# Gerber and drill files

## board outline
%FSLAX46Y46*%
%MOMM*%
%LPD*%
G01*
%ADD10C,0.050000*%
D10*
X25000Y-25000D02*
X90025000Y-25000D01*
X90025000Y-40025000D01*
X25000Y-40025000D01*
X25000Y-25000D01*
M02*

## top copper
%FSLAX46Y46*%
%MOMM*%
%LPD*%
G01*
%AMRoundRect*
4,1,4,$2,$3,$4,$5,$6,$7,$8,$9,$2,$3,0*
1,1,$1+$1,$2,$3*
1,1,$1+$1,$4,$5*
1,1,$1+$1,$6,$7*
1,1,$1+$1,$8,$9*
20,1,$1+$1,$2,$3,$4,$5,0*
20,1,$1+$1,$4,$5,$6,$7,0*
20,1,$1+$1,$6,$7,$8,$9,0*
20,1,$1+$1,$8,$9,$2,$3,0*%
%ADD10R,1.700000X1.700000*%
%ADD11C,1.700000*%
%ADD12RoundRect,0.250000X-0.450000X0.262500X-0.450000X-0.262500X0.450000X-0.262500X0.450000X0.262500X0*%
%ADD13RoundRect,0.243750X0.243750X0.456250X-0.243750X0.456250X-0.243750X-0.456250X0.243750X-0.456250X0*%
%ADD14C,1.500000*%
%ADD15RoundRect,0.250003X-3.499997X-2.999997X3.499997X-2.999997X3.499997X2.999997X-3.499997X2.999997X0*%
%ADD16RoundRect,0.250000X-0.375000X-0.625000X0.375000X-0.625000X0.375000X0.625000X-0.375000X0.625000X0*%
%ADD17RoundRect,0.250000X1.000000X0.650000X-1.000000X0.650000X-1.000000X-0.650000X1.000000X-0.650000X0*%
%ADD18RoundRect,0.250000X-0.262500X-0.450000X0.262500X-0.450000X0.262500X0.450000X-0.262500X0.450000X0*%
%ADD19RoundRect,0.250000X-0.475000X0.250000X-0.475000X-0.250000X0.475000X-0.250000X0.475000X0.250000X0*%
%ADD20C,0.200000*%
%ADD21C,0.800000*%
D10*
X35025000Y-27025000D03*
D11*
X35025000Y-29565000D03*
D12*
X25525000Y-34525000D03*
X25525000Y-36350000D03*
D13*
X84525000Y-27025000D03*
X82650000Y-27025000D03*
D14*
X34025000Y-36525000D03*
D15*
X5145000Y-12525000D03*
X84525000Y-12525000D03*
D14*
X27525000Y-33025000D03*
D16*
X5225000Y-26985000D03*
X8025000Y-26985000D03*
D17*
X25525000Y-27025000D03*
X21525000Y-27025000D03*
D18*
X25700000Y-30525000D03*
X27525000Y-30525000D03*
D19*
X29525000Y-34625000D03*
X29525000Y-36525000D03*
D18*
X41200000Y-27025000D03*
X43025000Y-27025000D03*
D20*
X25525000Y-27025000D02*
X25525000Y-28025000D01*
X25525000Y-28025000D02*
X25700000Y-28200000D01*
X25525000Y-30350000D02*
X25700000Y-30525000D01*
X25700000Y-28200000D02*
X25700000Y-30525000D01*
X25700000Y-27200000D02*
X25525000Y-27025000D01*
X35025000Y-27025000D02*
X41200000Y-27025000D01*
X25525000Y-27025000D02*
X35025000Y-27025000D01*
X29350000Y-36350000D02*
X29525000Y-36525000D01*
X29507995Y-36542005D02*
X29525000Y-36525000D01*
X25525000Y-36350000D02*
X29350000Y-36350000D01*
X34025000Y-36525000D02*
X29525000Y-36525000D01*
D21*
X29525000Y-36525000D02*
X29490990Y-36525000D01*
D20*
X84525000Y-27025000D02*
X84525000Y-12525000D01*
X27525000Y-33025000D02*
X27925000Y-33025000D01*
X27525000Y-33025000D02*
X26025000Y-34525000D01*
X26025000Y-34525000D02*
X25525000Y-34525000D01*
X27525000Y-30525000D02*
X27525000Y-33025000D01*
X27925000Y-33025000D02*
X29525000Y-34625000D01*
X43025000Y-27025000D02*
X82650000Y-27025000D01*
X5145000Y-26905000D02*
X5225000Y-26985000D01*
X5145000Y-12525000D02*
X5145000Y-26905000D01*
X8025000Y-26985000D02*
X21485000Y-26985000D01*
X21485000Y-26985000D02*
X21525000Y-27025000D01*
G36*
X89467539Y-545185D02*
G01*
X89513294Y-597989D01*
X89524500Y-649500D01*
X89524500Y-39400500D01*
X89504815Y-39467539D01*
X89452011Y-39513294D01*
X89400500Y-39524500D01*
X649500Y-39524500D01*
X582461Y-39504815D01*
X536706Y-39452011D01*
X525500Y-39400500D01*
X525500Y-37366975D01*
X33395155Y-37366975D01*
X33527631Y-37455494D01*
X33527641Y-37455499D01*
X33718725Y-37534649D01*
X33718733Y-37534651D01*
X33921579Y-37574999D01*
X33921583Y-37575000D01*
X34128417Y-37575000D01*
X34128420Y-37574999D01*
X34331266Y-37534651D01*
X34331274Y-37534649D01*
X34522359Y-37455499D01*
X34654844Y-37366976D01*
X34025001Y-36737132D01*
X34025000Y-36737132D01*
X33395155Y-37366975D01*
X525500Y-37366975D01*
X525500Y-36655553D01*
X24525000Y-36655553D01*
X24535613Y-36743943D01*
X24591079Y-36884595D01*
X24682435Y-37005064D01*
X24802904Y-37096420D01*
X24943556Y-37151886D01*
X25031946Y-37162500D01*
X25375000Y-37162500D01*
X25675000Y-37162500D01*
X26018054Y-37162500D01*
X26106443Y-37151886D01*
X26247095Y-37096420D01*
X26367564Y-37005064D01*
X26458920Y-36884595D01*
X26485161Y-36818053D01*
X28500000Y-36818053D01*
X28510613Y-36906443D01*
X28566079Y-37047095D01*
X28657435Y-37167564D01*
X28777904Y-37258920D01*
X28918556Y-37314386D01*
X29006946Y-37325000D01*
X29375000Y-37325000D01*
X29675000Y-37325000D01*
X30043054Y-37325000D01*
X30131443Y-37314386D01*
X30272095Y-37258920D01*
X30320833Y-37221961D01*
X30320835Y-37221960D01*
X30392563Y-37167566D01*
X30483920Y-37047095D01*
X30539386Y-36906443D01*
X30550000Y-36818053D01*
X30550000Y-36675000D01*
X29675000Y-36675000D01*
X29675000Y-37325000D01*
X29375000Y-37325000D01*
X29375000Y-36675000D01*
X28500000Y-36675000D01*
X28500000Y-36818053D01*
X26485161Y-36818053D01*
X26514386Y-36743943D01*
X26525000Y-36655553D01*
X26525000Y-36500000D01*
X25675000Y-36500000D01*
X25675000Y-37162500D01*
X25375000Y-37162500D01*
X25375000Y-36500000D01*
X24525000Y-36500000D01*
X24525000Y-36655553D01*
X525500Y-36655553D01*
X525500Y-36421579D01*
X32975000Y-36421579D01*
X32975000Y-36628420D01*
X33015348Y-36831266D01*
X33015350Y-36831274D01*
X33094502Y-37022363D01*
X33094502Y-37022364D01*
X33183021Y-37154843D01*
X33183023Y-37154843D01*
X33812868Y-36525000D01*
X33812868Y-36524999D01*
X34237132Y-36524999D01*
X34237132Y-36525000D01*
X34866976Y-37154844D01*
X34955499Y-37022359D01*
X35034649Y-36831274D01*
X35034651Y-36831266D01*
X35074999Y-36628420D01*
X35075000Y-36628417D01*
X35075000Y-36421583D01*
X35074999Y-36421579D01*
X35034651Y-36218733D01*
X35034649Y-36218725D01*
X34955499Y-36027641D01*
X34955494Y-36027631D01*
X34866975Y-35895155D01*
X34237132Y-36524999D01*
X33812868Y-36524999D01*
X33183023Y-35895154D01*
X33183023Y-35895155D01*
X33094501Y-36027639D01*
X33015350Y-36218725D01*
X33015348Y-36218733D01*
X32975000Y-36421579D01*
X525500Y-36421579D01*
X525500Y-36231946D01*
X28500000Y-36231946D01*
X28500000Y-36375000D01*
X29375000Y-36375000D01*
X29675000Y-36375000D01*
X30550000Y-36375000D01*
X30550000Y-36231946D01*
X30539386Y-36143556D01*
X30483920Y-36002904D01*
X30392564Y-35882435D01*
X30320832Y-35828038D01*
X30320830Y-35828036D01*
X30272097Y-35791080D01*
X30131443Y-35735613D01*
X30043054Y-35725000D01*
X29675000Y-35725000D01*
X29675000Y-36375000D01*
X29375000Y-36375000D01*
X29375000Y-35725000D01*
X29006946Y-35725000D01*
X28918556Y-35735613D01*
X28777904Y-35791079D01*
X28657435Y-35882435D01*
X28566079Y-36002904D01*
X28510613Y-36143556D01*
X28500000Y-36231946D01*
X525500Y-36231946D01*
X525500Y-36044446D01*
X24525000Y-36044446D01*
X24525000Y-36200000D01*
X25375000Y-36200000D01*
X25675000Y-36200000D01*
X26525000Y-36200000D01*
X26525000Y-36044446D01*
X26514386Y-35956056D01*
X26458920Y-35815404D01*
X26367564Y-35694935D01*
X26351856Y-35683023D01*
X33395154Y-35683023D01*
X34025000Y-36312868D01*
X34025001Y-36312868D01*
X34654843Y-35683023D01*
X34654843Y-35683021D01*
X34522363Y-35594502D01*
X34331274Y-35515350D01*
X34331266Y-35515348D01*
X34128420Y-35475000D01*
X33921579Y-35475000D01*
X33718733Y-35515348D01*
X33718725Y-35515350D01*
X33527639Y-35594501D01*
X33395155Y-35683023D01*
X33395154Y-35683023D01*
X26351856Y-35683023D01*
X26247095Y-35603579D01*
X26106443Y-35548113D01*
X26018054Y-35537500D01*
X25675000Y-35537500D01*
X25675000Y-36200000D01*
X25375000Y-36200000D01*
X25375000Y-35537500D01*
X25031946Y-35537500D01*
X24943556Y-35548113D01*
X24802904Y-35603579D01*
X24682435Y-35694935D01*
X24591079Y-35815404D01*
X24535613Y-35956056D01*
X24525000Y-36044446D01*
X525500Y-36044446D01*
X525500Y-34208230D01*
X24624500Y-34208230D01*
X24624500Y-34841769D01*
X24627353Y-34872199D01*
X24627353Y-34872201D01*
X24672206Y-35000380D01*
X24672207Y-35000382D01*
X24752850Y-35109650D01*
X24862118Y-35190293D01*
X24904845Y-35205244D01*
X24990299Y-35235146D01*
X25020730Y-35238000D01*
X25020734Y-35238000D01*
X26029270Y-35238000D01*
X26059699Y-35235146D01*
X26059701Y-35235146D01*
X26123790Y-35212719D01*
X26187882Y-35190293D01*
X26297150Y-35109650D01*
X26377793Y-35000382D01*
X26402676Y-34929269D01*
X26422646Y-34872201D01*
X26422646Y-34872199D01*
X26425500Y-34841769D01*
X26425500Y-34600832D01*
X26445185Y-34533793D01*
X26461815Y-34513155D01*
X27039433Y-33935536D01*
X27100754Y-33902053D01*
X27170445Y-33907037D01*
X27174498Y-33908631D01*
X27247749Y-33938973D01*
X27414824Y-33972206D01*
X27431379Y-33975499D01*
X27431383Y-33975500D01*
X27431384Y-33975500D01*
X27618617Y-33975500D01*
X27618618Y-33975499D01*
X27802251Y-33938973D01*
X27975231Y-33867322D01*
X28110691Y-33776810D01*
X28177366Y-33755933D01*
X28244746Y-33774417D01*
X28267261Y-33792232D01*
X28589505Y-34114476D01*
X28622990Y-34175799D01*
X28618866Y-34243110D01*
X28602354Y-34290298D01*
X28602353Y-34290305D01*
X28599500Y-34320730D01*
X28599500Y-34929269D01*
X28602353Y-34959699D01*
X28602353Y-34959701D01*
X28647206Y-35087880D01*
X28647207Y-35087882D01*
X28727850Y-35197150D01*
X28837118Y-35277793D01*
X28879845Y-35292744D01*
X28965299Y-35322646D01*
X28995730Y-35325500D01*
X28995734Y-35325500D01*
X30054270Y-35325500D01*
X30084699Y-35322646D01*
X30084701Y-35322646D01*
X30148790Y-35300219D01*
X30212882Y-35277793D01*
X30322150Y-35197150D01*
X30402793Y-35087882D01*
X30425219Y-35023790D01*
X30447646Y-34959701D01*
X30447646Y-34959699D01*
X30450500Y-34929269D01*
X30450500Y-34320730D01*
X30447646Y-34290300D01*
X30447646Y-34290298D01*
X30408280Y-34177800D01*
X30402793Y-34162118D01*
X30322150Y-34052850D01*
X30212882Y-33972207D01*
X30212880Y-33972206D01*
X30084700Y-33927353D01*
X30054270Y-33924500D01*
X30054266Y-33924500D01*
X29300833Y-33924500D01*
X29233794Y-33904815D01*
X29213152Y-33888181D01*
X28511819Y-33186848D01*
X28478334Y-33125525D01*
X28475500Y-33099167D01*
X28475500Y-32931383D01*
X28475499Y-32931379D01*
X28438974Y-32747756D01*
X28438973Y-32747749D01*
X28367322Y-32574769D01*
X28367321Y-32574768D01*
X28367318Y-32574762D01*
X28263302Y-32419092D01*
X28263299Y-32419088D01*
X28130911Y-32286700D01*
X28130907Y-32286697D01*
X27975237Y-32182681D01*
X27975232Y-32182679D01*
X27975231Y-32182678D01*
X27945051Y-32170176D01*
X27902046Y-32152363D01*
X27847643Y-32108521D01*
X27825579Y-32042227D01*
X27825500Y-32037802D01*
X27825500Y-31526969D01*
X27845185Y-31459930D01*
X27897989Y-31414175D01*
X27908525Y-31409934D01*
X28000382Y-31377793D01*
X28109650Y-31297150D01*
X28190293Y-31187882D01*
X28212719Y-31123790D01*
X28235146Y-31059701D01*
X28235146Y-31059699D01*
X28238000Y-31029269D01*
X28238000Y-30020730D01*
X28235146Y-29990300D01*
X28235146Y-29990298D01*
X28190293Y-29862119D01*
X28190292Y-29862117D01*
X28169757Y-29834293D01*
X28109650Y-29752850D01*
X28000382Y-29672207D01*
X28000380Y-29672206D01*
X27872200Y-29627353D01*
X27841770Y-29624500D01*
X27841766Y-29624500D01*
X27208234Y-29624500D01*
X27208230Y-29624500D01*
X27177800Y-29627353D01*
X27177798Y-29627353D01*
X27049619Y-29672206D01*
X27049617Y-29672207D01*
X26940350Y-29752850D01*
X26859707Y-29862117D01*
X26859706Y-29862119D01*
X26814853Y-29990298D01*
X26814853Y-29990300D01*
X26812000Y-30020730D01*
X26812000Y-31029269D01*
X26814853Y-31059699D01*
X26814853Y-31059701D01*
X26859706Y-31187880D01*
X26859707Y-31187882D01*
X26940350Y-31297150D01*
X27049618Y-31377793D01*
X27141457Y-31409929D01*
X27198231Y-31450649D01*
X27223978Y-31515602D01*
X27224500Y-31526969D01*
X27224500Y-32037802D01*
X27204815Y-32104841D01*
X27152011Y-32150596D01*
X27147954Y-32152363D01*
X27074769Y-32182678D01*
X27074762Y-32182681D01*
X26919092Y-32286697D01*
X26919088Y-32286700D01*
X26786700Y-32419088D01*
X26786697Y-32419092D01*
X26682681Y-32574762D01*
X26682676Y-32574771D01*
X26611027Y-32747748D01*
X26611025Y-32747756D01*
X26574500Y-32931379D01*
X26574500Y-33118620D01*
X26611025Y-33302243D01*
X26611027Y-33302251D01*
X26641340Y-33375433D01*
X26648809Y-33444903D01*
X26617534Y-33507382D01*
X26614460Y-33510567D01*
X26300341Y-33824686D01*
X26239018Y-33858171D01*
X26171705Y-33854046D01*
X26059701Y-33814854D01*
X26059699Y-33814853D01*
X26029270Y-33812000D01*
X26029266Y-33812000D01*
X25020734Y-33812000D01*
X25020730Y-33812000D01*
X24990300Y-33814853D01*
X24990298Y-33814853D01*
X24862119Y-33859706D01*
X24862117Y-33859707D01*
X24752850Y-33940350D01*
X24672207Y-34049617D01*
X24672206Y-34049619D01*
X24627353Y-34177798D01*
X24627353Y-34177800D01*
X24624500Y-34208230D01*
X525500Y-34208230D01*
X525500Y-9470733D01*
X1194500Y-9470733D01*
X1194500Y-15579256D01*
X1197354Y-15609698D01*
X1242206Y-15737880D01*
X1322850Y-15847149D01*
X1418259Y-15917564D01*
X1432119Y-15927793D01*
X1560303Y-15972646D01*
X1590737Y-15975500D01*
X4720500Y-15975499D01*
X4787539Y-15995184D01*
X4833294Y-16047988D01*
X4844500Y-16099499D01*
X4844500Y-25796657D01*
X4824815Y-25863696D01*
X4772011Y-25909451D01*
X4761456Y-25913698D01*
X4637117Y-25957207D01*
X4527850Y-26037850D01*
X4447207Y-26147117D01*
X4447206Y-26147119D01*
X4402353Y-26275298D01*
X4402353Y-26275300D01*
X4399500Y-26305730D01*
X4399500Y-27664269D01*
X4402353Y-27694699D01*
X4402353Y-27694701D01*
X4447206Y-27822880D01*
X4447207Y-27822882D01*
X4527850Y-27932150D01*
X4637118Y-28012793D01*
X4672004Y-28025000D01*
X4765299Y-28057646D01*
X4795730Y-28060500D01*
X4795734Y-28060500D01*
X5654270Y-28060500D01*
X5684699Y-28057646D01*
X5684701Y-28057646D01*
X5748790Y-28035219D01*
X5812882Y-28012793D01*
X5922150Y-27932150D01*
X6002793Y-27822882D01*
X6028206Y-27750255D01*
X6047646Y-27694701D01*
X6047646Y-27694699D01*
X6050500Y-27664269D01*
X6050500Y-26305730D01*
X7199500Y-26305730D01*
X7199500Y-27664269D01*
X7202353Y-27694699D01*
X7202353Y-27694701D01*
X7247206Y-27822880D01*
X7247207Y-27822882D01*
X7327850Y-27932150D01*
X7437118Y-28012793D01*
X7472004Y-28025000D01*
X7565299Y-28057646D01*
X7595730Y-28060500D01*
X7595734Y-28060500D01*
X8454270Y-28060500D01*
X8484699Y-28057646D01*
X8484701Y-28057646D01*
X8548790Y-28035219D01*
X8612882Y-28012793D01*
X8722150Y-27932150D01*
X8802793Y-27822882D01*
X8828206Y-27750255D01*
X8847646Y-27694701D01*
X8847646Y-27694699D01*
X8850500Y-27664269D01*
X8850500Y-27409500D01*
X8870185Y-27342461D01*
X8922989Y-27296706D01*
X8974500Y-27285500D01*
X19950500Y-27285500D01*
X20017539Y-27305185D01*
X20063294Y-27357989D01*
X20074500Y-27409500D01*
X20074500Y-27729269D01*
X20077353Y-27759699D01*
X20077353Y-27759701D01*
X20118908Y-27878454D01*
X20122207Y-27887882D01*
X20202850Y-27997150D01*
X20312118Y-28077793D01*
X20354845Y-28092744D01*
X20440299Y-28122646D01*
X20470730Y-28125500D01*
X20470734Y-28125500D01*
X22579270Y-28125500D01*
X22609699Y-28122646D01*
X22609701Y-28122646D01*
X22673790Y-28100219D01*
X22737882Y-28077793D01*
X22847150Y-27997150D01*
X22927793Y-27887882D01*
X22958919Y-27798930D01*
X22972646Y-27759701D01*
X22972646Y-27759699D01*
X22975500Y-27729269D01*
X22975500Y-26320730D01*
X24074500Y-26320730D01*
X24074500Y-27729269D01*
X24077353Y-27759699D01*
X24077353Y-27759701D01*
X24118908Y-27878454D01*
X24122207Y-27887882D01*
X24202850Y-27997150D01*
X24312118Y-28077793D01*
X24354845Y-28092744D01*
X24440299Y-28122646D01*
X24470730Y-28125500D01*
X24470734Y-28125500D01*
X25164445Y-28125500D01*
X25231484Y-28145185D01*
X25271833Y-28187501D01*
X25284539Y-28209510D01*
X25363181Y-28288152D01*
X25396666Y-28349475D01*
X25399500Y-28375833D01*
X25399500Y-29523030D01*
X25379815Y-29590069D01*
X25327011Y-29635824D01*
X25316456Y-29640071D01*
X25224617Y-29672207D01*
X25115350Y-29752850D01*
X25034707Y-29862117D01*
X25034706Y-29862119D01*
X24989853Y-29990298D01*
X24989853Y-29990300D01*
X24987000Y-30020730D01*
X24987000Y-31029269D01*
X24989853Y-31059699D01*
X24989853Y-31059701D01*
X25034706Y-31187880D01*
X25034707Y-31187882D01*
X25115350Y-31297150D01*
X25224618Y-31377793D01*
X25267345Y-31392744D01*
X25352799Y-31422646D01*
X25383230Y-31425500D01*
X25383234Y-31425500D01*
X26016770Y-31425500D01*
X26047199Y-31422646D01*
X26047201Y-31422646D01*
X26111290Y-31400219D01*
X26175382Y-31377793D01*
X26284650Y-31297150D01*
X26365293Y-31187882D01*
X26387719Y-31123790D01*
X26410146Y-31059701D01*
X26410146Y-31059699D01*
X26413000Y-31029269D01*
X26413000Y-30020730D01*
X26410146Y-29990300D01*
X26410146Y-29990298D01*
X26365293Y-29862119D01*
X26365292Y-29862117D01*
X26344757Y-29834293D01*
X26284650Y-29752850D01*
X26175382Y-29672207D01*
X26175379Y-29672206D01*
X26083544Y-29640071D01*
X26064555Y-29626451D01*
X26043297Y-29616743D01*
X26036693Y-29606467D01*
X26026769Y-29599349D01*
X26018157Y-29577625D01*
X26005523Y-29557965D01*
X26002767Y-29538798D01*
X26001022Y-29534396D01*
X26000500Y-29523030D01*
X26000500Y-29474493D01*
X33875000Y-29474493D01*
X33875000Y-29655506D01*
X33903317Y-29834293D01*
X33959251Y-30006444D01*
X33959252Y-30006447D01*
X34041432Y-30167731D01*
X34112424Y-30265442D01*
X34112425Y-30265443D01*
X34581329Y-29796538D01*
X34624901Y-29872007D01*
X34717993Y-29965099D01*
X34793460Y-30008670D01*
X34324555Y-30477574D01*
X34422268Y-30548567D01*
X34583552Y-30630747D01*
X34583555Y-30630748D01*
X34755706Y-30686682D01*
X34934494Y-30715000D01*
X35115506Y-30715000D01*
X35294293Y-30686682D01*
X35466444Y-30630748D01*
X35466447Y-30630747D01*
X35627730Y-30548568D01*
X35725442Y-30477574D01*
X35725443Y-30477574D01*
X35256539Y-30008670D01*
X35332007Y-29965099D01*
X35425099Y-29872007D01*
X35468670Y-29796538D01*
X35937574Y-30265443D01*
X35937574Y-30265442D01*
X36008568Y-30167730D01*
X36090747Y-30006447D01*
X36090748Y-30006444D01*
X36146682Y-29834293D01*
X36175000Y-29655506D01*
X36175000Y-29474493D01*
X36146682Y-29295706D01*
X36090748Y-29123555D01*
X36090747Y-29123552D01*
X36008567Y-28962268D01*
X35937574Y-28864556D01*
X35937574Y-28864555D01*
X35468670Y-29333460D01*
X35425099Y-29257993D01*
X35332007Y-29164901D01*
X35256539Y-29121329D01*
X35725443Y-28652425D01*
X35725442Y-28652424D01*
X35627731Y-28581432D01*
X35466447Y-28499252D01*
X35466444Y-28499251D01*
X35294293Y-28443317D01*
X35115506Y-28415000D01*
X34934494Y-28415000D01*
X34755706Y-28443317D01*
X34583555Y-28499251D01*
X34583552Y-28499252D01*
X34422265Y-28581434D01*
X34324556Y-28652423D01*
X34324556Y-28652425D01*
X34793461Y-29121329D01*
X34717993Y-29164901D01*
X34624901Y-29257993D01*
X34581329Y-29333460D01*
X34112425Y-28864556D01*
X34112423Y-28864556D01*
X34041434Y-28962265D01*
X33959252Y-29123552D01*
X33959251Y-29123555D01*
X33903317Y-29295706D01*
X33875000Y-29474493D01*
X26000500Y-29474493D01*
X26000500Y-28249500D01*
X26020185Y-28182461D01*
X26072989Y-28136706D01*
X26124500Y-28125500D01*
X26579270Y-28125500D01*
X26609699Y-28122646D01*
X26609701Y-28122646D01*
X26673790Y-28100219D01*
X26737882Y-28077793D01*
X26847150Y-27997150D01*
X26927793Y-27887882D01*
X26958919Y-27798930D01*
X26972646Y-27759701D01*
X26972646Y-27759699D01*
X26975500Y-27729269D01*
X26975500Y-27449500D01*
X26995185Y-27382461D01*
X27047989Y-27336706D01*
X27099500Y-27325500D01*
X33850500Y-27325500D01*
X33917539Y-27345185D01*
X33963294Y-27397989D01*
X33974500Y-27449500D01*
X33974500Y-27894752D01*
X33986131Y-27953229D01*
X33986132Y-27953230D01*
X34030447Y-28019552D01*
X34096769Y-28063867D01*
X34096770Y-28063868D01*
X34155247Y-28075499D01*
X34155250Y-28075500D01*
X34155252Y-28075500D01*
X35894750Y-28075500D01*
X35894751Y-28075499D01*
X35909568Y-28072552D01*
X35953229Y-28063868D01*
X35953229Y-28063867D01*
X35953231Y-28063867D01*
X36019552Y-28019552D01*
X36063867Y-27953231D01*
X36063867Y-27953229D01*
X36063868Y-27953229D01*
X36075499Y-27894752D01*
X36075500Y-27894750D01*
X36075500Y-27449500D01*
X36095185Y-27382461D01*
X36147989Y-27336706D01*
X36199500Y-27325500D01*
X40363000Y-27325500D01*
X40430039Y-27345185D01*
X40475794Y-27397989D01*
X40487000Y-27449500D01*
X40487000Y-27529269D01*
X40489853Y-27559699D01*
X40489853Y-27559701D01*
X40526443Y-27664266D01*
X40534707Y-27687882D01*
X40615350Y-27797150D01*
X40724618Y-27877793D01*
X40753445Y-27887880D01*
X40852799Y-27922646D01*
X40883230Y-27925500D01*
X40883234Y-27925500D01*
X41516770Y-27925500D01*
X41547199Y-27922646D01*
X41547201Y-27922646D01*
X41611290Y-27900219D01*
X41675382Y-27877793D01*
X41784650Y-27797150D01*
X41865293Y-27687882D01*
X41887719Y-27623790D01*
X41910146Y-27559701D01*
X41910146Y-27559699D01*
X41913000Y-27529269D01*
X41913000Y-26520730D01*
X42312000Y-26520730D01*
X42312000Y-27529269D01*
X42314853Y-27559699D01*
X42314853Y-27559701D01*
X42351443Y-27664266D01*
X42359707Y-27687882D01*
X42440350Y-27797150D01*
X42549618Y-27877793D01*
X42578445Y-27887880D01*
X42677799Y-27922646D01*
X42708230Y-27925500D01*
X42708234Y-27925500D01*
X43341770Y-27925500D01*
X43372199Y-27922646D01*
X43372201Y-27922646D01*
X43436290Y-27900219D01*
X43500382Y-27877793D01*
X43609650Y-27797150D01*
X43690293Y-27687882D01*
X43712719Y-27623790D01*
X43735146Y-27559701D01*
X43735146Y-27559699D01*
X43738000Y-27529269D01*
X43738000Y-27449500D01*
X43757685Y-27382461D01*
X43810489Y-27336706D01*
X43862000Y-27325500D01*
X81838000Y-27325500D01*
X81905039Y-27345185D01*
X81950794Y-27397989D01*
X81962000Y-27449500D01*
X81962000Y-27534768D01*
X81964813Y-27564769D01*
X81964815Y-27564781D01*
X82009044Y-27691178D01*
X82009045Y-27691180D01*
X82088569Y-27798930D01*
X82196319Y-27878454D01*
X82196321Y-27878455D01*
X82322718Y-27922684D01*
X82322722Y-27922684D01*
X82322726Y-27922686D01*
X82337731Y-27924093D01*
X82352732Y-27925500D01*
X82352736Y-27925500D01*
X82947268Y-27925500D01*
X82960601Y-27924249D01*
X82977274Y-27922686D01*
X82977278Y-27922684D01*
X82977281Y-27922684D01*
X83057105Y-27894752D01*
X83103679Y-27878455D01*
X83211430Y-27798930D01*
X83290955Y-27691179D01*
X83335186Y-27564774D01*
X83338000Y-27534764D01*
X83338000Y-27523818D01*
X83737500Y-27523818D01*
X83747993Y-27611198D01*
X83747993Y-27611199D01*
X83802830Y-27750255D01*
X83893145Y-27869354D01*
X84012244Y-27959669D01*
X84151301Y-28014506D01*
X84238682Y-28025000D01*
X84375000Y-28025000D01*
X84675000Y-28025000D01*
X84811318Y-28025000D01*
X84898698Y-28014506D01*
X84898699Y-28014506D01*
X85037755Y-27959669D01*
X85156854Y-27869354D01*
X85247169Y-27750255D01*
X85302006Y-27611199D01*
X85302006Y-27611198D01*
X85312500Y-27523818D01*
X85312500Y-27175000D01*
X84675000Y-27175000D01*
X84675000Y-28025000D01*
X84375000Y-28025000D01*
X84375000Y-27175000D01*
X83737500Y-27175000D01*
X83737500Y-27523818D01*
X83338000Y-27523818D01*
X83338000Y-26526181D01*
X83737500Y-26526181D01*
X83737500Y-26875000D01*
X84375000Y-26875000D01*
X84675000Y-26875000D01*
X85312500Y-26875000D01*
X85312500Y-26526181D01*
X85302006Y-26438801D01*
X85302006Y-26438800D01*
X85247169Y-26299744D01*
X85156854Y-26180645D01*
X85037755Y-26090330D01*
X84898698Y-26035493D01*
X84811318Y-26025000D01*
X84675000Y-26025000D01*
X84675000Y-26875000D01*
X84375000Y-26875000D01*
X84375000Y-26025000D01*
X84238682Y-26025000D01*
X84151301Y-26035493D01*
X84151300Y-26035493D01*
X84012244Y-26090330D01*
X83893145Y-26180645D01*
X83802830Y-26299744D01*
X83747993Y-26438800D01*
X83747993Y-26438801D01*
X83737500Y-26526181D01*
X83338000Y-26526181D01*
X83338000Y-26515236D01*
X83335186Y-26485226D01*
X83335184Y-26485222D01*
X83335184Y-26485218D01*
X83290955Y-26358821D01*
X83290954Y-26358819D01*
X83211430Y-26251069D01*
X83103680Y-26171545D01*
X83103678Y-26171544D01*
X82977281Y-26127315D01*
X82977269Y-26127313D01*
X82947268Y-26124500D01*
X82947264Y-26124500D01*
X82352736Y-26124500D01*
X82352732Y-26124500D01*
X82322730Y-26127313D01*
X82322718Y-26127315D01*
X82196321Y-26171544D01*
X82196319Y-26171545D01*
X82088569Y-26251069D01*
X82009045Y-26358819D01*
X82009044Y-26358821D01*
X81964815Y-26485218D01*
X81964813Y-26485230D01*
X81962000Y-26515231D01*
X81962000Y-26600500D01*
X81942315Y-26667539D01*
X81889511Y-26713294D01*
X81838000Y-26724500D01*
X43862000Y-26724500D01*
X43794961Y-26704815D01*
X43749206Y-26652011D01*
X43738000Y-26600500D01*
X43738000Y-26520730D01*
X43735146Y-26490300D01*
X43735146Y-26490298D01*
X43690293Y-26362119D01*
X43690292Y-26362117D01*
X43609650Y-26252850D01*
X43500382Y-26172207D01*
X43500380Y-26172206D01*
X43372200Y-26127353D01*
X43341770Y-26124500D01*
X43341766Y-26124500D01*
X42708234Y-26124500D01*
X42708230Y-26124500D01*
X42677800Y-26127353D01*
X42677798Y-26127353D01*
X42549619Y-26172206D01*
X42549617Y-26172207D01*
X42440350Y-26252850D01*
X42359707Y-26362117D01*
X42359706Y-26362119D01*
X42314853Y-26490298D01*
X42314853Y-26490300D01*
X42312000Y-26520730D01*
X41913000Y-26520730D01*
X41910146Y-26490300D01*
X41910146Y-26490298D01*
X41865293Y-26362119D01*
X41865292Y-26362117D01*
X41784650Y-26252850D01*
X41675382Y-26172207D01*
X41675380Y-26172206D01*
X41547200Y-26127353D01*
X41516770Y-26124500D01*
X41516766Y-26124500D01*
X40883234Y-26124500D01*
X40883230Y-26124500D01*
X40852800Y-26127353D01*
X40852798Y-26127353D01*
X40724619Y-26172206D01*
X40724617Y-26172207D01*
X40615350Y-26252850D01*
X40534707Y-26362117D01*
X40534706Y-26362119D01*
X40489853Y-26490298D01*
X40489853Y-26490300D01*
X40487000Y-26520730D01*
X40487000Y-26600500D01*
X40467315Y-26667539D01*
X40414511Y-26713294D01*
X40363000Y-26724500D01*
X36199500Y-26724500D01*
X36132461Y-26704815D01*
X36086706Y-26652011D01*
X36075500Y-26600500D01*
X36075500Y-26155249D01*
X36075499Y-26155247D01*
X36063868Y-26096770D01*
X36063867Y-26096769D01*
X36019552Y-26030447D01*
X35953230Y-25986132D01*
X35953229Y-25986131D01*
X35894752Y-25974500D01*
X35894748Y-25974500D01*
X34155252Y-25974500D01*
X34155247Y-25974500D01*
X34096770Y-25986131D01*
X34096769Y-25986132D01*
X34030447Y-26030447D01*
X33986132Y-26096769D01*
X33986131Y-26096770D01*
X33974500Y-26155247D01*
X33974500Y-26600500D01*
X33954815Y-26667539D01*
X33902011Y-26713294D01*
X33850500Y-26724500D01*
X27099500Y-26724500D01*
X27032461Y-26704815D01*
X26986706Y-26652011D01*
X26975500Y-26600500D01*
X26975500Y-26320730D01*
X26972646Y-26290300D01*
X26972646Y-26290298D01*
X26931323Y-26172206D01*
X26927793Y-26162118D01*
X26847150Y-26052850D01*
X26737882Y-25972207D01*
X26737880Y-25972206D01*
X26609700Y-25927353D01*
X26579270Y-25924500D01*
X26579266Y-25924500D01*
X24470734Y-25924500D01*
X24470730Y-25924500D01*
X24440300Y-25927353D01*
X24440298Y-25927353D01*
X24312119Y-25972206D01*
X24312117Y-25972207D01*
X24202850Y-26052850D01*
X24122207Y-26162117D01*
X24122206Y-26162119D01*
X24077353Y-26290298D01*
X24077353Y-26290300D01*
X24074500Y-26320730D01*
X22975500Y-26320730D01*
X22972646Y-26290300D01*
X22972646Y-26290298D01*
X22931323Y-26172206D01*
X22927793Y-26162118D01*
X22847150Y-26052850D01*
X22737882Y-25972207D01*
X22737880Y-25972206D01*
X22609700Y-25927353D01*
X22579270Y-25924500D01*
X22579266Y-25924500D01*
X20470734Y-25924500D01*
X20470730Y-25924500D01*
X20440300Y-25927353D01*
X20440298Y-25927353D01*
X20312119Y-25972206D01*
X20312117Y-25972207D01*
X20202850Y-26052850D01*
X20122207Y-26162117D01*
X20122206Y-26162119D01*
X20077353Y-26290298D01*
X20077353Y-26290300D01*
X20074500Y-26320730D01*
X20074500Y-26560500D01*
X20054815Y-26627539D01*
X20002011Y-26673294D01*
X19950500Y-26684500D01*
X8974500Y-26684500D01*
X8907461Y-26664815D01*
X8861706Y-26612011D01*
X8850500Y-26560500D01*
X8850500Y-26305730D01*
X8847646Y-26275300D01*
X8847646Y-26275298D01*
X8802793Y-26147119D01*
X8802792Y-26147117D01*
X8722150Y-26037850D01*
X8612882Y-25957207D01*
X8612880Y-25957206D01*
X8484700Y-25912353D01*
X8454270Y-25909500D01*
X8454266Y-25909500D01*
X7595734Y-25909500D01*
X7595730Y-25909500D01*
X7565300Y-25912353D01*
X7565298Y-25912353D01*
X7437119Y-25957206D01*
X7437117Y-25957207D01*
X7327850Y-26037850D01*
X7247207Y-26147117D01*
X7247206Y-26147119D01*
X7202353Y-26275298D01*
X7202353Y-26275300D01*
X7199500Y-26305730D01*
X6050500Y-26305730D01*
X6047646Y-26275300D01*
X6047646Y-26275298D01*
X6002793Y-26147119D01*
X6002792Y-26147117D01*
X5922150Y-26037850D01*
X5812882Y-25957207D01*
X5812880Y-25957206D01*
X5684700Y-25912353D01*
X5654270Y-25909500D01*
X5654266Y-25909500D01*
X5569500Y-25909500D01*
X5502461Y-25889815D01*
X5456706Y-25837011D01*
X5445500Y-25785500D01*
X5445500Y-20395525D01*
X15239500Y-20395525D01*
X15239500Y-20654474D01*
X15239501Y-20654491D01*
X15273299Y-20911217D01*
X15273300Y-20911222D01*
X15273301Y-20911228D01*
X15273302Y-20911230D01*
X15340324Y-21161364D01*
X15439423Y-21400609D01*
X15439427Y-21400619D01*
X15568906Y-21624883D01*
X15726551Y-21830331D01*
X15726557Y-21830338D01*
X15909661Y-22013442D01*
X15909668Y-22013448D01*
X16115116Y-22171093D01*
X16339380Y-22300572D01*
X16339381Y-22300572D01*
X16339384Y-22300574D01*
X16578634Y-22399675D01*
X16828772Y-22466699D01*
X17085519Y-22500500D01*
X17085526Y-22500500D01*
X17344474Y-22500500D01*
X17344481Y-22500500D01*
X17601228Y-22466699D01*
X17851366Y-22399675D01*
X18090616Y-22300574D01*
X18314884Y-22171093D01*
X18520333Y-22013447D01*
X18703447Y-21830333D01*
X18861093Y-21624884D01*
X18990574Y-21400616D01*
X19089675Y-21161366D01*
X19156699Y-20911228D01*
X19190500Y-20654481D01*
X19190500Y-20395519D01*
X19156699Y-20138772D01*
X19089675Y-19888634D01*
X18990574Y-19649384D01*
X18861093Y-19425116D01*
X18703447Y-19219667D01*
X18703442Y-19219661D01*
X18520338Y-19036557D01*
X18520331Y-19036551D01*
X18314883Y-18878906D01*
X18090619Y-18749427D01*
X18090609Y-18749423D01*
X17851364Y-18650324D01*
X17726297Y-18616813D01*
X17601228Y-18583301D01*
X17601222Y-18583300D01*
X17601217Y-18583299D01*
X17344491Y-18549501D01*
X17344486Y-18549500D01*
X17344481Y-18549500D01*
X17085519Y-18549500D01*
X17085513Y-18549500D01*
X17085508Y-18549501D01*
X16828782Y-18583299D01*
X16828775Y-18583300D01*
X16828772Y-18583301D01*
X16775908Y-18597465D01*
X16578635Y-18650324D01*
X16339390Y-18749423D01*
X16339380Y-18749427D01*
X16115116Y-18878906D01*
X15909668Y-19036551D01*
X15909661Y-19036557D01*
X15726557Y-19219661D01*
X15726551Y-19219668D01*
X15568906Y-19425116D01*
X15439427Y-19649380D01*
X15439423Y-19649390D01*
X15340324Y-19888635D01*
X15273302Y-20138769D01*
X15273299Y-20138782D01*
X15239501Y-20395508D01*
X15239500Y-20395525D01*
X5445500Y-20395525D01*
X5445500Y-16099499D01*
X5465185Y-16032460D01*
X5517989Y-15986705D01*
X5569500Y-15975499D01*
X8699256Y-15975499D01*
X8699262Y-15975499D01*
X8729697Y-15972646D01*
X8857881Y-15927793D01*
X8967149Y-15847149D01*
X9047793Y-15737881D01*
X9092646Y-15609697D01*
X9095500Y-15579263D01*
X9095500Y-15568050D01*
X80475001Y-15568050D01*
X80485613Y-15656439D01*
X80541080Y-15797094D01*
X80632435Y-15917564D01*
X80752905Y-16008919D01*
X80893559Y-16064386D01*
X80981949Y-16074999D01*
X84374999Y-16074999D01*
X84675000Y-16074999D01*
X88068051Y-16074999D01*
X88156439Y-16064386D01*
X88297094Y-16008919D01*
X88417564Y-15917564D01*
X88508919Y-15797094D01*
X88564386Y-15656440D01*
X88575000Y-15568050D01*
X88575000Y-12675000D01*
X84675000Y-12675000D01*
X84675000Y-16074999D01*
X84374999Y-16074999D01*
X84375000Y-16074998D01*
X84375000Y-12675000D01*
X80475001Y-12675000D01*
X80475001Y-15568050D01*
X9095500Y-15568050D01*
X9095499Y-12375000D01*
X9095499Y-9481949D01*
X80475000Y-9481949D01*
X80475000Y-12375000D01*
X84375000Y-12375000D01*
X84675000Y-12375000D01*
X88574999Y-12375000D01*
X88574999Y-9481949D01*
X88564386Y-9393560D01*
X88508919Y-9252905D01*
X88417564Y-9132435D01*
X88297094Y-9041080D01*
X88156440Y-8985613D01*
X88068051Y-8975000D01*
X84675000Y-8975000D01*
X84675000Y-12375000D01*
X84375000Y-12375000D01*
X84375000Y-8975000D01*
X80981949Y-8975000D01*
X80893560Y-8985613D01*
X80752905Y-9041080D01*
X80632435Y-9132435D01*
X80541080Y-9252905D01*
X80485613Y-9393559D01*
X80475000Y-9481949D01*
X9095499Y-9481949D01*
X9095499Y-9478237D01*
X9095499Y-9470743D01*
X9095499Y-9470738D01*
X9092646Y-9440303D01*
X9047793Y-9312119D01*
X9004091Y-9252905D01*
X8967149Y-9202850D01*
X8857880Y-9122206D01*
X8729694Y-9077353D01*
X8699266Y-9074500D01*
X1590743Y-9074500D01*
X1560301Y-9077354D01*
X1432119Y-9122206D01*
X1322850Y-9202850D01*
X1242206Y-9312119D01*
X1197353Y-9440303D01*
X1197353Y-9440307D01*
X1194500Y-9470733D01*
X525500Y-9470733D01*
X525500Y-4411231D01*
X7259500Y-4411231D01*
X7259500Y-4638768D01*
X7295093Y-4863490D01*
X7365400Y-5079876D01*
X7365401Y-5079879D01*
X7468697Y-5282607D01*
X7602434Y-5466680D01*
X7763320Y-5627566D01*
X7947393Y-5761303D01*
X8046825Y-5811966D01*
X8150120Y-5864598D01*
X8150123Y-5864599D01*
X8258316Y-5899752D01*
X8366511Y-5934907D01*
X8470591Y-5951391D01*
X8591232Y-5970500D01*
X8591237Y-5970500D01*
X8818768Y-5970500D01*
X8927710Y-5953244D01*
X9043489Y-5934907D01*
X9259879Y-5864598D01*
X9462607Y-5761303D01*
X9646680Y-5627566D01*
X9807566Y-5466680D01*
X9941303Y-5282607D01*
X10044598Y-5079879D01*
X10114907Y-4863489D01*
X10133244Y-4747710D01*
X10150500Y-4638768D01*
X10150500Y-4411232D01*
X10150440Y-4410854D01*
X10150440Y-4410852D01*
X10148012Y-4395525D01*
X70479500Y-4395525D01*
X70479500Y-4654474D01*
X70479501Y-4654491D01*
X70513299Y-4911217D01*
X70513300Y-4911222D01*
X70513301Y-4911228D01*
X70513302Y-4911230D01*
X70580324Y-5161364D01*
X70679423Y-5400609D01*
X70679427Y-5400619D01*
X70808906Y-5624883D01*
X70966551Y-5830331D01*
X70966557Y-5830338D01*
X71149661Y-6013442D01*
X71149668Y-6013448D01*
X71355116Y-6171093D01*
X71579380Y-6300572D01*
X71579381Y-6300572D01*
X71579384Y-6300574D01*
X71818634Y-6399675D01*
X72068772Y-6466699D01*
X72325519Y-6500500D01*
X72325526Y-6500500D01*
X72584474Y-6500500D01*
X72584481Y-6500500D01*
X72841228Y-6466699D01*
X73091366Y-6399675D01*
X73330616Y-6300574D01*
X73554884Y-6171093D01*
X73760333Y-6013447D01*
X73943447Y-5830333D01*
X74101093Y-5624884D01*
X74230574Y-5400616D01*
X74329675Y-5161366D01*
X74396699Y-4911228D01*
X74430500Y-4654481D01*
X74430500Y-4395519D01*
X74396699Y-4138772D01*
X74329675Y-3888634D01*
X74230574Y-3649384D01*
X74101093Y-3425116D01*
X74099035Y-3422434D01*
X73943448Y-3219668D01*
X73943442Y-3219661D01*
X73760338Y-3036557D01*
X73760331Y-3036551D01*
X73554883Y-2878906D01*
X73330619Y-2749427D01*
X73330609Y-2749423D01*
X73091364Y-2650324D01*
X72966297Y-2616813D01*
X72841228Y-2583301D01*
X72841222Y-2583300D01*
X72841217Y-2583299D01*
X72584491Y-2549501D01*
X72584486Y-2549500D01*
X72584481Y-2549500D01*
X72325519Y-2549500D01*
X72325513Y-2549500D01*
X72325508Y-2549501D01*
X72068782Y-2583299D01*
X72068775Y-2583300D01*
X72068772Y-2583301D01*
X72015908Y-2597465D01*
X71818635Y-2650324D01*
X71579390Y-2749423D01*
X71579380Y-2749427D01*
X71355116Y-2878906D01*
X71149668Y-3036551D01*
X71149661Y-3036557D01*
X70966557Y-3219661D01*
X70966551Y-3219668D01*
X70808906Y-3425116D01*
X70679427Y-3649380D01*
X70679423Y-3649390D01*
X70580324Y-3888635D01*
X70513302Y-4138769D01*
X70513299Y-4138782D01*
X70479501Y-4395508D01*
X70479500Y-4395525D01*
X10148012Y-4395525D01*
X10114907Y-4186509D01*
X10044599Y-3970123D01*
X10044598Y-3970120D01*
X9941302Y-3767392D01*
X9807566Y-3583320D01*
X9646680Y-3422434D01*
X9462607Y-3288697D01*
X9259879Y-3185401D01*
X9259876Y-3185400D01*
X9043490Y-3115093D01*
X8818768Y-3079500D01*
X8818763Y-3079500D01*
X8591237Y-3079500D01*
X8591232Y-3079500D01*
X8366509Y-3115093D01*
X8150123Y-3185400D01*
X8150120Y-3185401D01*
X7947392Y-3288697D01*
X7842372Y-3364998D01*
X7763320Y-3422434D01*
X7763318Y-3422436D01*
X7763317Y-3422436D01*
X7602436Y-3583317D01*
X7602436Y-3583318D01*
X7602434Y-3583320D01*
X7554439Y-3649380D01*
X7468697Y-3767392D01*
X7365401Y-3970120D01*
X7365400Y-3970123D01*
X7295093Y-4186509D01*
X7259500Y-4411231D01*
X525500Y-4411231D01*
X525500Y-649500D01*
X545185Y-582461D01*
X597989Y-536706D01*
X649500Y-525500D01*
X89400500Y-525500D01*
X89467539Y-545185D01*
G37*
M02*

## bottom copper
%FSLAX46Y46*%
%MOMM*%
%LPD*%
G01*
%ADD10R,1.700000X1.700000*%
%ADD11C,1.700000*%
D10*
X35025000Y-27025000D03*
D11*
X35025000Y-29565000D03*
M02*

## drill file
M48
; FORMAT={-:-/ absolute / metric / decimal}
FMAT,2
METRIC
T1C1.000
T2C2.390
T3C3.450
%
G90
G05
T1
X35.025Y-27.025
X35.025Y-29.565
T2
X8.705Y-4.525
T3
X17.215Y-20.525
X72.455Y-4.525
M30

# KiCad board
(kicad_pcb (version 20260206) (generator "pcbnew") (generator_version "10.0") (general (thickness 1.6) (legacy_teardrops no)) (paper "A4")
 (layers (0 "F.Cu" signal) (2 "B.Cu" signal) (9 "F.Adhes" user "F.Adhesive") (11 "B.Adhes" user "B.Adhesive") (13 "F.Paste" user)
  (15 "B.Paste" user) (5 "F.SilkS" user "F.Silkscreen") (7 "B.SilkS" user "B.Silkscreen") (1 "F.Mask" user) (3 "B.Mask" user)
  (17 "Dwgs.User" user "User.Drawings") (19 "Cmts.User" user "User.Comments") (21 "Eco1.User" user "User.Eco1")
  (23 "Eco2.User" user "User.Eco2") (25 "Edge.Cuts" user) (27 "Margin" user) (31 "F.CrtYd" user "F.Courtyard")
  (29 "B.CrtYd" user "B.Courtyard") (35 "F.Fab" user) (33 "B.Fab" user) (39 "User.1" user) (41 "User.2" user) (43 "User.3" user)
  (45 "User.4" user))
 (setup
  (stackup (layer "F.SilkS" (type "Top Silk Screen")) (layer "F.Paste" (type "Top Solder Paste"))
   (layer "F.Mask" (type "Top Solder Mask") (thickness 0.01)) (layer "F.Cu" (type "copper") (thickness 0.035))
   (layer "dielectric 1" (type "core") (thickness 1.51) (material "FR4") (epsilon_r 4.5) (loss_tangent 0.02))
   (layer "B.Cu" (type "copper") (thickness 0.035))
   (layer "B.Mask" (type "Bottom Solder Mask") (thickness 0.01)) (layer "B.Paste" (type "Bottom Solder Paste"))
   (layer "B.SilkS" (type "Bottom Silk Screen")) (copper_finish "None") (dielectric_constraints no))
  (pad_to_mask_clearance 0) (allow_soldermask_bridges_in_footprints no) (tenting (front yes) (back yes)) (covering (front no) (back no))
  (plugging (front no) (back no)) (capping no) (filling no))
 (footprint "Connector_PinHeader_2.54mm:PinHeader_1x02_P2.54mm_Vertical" (layer "F.Cu") (at 35.025 27.025)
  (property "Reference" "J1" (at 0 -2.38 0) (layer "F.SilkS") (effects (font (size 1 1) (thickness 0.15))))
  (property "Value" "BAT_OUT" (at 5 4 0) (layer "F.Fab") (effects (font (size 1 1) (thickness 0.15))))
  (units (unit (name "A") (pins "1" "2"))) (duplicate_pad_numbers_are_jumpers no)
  (pad "1" thru_hole rect (at 0 0) (size 1.7 1.7) (drill 1) (layers "*.Cu" "*.Mask") (remove_unused_layers no) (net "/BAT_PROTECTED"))
  (pad "2" thru_hole circle (at 0 2.54) (size 1.7 1.7) (drill 1) (layers "*.Cu" "*.Mask") (remove_unused_layers no) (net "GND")))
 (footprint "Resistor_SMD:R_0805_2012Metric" (layer "F.Cu") (at 25.525 35.4375 -90)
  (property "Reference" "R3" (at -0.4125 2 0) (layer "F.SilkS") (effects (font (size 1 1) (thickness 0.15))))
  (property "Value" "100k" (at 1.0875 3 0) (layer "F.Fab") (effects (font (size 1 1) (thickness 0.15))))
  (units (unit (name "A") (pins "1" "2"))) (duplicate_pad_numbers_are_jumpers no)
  (pad "1" smd roundrect (at -0.9125 0 270) (size 1.025 1.4) (layers "F.Cu" "F.Mask" "F.Paste") (roundrect_rratio 0.243902)
   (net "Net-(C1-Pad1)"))
  (pad "2" smd roundrect (at 0.9125 0 270) (size 1.025 1.4) (layers "F.Cu" "F.Mask" "F.Paste") (roundrect_rratio 0.243902) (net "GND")))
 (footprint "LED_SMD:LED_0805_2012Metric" (layer "F.Cu") (at 83.5875 27.025 180)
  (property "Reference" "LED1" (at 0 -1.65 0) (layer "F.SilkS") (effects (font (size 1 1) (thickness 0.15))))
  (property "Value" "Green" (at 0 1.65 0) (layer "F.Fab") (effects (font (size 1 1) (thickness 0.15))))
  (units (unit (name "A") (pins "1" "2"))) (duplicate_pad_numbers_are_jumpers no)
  (pad "1" smd roundrect (at -0.9375 0 180) (size 0.975 1.4) (layers "F.Cu" "F.Mask" "F.Paste") (roundrect_rratio 0.25) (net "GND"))
  (pad "2" smd roundrect (at 0.9375 0 180) (size 0.975 1.4) (layers "F.Cu" "F.Mask" "F.Paste") (roundrect_rratio 0.25) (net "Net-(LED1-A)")))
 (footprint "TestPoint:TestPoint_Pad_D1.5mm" (layer "F.Cu") (at 34.025 36.525)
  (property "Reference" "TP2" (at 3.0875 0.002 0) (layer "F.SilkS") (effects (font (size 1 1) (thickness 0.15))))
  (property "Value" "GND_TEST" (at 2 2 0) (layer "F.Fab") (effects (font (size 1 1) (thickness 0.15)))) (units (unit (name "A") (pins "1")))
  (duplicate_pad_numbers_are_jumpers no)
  (pad "1" smd circle (at 0 0) (size 1.5 1.5) (layers "F.Cu" "F.Mask") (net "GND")))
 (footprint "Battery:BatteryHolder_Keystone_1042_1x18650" (layer "F.Cu") (at 44.835 12.525)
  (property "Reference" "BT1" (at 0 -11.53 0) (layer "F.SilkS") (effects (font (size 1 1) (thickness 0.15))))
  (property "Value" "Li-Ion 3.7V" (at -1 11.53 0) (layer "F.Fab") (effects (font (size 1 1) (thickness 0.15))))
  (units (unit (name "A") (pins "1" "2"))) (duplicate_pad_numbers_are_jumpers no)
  (pad "" np_thru_hole circle (at -36.13 -8) (size 2.39 2.39) (drill 2.39) (layers "*.Cu" "*.Mask"))
  (pad "" np_thru_hole circle (at -27.62 8) (size 3.45 3.45) (drill 3.45) (layers "*.Cu" "*.Mask"))
  (pad "" np_thru_hole circle (at 27.62 -8) (size 3.45 3.45) (drill 3.45) (layers "*.Cu" "*.Mask"))
  (pad "1" smd roundrect (at -39.69 0) (size 7.5 6.5) (layers "F.Cu" "F.Mask" "F.Paste") (roundrect_rratio 0.038462) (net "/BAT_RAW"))
  (pad "2" smd roundrect (at 39.69 0) (size 7.5 6.5) (layers "F.Cu" "F.Mask" "F.Paste") (roundrect_rratio 0.038462) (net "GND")))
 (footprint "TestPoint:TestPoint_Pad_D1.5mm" (layer "F.Cu") (at 27.525 33.025)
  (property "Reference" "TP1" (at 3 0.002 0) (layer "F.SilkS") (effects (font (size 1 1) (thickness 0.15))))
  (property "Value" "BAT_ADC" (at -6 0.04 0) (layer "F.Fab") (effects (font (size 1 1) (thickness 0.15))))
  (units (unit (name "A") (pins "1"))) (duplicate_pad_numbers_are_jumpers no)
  (pad "1" smd circle (at 0 0) (size 1.5 1.5) (layers "F.Cu" "F.Mask") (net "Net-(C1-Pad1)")))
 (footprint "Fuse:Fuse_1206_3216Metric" (layer "F.Cu") (at 6.625 26.985)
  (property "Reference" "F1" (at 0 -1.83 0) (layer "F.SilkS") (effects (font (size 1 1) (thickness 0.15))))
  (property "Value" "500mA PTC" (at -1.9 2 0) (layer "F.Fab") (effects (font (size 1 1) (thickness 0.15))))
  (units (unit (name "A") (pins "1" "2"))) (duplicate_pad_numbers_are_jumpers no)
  (pad "1" smd roundrect (at -1.4 0) (size 1.25 1.75) (layers "F.Cu" "F.Mask" "F.Paste") (roundrect_rratio 0.2) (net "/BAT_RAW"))
  (pad "2" smd roundrect (at 1.4 0) (size 1.25 1.75) (layers "F.Cu" "F.Mask" "F.Paste") (roundrect_rratio 0.2) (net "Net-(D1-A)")))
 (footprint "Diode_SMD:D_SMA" (layer "F.Cu") (at 23.525 27.025 180)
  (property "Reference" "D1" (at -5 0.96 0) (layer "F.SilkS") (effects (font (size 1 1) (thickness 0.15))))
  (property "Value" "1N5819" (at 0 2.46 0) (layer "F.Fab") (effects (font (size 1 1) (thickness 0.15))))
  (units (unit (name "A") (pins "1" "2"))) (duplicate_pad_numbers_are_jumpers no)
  (pad "1" smd roundrect (at -2 0 180) (size 2.5 1.8) (layers "F.Cu" "F.Mask" "F.Paste") (roundrect_rratio 0.1388888889)
   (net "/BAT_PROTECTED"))
  (pad "2" smd roundrect (at 2 0 180) (size 2.5 1.8) (layers "F.Cu" "F.Mask" "F.Paste") (roundrect_rratio 0.1388888889) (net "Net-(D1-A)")))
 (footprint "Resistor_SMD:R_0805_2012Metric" (layer "F.Cu") (at 26.6125 30.525)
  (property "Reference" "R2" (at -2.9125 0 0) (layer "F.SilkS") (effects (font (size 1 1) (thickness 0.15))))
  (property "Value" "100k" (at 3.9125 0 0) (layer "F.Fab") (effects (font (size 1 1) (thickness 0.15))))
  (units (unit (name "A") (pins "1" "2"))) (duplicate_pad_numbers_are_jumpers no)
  (pad "1" smd roundrect (at -0.9125 0) (size 1.025 1.4) (layers "F.Cu" "F.Mask" "F.Paste") (roundrect_rratio 0.243902)
   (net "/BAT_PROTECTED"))
  (pad "2" smd roundrect (at 0.9125 0) (size 1.025 1.4) (layers "F.Cu" "F.Mask" "F.Paste") (roundrect_rratio 0.243902) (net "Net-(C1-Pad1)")))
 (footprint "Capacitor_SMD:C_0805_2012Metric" (layer "F.Cu") (at 29.525 35.575 -90)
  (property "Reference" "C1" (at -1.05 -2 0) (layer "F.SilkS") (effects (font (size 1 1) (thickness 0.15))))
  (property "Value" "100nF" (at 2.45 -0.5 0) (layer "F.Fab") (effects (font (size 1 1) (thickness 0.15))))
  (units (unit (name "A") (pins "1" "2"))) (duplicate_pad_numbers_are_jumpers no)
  (pad "1" smd roundrect (at -0.95 0 270) (size 1 1.45) (layers "F.Cu" "F.Mask" "F.Paste") (roundrect_rratio 0.25) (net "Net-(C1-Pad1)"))
  (pad "2" smd roundrect (at 0.95 0 270) (size 1 1.45) (layers "F.Cu" "F.Mask" "F.Paste") (roundrect_rratio 0.25) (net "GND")))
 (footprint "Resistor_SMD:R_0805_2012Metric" (layer "F.Cu") (at 42.1125 27.025)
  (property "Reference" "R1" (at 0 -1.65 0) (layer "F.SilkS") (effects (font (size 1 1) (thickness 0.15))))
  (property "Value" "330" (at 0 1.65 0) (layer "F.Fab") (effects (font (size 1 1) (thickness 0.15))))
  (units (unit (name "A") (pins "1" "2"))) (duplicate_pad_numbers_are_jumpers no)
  (pad "1" smd roundrect (at -0.9125 0) (size 1.025 1.4) (layers "F.Cu" "F.Mask" "F.Paste") (roundrect_rratio 0.243902)
   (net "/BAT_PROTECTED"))
  (pad "2" smd roundrect (at 0.9125 0) (size 1.025 1.4) (layers "F.Cu" "F.Mask" "F.Paste") (roundrect_rratio 0.243902) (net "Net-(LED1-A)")))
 (gr_rect (start 0.025 0.025) (end 90.025 40.025) (stroke (width 0.05) (type default)) (fill no) (layer "Edge.Cuts"))
 (segment (start 25.525 27.025) (end 25.525 28.025) (width 0.2) (layer "F.Cu") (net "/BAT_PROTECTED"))
 (segment (start 25.525 28.025) (end 25.7 28.2) (width 0.2) (layer "F.Cu") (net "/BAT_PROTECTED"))
 (segment (start 25.525 30.35) (end 25.7 30.525) (width 0.2) (layer "F.Cu") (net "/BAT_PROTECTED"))
 (segment (start 25.7 28.2) (end 25.7 30.525) (width 0.2) (layer "F.Cu") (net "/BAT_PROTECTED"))
 (segment (start 25.7 27.2) (end 25.525 27.025) (width 0.2) (layer "F.Cu") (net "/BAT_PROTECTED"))
 (segment (start 35.025 27.025) (end 41.2 27.025) (width 0.2) (layer "F.Cu") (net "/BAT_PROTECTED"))
 (segment (start 25.525 27.025) (end 35.025 27.025) (width 0.2) (layer "F.Cu") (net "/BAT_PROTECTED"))
 (segment (start 29.35 36.35) (end 29.525 36.525) (width 0.2) (layer "F.Cu") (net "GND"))
 (segment (start 29.507995 36.542005) (end 29.525 36.525) (width 0.2) (layer "F.Cu") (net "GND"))
 (segment (start 25.525 36.35) (end 29.35 36.35) (width 0.2) (layer "F.Cu") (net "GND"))
 (segment (start 34.025 36.525) (end 29.525 36.525) (width 0.2) (layer "F.Cu") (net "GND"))
 (segment (start 29.525 36.525) (end 29.49099 36.525) (width 0.8) (layer "F.Cu") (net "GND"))
 (segment (start 84.525 27.025) (end 84.525 12.525) (width 0.2) (layer "F.Cu") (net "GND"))
 (segment (start 27.525 33.025) (end 27.925 33.025) (width 0.2) (layer "F.Cu") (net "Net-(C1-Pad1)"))
 (segment (start 27.525 33.025) (end 26.025 34.525) (width 0.2) (layer "F.Cu") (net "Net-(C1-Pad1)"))
 (segment (start 26.025 34.525) (end 25.525 34.525) (width 0.2) (layer "F.Cu") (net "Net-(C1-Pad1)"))
 (segment (start 27.525 30.525) (end 27.525 33.025) (width 0.2) (layer "F.Cu") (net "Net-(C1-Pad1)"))
 (segment (start 27.925 33.025) (end 29.525 34.625) (width 0.2) (layer "F.Cu") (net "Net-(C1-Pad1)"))
 (segment (start 43.025 27.025) (end 82.65 27.025) (width 0.2) (layer "F.Cu") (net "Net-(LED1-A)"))
 (segment (start 5.145 26.905) (end 5.225 26.985) (width 0.2) (layer "F.Cu") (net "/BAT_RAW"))
 (segment (start 5.145 12.525) (end 5.145 26.905) (width 0.2) (layer "F.Cu") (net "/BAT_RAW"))
 (segment (start 8.025 26.985) (end 21.485 26.985) (width 0.2) (layer "F.Cu") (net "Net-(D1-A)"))
 (segment (start 21.485 26.985) (end 21.525 27.025) (width 0.2) (layer "F.Cu") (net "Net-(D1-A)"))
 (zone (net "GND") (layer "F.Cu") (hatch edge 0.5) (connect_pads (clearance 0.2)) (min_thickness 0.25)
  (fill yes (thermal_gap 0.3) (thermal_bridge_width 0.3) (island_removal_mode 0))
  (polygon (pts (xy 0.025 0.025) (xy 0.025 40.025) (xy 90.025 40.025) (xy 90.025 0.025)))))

